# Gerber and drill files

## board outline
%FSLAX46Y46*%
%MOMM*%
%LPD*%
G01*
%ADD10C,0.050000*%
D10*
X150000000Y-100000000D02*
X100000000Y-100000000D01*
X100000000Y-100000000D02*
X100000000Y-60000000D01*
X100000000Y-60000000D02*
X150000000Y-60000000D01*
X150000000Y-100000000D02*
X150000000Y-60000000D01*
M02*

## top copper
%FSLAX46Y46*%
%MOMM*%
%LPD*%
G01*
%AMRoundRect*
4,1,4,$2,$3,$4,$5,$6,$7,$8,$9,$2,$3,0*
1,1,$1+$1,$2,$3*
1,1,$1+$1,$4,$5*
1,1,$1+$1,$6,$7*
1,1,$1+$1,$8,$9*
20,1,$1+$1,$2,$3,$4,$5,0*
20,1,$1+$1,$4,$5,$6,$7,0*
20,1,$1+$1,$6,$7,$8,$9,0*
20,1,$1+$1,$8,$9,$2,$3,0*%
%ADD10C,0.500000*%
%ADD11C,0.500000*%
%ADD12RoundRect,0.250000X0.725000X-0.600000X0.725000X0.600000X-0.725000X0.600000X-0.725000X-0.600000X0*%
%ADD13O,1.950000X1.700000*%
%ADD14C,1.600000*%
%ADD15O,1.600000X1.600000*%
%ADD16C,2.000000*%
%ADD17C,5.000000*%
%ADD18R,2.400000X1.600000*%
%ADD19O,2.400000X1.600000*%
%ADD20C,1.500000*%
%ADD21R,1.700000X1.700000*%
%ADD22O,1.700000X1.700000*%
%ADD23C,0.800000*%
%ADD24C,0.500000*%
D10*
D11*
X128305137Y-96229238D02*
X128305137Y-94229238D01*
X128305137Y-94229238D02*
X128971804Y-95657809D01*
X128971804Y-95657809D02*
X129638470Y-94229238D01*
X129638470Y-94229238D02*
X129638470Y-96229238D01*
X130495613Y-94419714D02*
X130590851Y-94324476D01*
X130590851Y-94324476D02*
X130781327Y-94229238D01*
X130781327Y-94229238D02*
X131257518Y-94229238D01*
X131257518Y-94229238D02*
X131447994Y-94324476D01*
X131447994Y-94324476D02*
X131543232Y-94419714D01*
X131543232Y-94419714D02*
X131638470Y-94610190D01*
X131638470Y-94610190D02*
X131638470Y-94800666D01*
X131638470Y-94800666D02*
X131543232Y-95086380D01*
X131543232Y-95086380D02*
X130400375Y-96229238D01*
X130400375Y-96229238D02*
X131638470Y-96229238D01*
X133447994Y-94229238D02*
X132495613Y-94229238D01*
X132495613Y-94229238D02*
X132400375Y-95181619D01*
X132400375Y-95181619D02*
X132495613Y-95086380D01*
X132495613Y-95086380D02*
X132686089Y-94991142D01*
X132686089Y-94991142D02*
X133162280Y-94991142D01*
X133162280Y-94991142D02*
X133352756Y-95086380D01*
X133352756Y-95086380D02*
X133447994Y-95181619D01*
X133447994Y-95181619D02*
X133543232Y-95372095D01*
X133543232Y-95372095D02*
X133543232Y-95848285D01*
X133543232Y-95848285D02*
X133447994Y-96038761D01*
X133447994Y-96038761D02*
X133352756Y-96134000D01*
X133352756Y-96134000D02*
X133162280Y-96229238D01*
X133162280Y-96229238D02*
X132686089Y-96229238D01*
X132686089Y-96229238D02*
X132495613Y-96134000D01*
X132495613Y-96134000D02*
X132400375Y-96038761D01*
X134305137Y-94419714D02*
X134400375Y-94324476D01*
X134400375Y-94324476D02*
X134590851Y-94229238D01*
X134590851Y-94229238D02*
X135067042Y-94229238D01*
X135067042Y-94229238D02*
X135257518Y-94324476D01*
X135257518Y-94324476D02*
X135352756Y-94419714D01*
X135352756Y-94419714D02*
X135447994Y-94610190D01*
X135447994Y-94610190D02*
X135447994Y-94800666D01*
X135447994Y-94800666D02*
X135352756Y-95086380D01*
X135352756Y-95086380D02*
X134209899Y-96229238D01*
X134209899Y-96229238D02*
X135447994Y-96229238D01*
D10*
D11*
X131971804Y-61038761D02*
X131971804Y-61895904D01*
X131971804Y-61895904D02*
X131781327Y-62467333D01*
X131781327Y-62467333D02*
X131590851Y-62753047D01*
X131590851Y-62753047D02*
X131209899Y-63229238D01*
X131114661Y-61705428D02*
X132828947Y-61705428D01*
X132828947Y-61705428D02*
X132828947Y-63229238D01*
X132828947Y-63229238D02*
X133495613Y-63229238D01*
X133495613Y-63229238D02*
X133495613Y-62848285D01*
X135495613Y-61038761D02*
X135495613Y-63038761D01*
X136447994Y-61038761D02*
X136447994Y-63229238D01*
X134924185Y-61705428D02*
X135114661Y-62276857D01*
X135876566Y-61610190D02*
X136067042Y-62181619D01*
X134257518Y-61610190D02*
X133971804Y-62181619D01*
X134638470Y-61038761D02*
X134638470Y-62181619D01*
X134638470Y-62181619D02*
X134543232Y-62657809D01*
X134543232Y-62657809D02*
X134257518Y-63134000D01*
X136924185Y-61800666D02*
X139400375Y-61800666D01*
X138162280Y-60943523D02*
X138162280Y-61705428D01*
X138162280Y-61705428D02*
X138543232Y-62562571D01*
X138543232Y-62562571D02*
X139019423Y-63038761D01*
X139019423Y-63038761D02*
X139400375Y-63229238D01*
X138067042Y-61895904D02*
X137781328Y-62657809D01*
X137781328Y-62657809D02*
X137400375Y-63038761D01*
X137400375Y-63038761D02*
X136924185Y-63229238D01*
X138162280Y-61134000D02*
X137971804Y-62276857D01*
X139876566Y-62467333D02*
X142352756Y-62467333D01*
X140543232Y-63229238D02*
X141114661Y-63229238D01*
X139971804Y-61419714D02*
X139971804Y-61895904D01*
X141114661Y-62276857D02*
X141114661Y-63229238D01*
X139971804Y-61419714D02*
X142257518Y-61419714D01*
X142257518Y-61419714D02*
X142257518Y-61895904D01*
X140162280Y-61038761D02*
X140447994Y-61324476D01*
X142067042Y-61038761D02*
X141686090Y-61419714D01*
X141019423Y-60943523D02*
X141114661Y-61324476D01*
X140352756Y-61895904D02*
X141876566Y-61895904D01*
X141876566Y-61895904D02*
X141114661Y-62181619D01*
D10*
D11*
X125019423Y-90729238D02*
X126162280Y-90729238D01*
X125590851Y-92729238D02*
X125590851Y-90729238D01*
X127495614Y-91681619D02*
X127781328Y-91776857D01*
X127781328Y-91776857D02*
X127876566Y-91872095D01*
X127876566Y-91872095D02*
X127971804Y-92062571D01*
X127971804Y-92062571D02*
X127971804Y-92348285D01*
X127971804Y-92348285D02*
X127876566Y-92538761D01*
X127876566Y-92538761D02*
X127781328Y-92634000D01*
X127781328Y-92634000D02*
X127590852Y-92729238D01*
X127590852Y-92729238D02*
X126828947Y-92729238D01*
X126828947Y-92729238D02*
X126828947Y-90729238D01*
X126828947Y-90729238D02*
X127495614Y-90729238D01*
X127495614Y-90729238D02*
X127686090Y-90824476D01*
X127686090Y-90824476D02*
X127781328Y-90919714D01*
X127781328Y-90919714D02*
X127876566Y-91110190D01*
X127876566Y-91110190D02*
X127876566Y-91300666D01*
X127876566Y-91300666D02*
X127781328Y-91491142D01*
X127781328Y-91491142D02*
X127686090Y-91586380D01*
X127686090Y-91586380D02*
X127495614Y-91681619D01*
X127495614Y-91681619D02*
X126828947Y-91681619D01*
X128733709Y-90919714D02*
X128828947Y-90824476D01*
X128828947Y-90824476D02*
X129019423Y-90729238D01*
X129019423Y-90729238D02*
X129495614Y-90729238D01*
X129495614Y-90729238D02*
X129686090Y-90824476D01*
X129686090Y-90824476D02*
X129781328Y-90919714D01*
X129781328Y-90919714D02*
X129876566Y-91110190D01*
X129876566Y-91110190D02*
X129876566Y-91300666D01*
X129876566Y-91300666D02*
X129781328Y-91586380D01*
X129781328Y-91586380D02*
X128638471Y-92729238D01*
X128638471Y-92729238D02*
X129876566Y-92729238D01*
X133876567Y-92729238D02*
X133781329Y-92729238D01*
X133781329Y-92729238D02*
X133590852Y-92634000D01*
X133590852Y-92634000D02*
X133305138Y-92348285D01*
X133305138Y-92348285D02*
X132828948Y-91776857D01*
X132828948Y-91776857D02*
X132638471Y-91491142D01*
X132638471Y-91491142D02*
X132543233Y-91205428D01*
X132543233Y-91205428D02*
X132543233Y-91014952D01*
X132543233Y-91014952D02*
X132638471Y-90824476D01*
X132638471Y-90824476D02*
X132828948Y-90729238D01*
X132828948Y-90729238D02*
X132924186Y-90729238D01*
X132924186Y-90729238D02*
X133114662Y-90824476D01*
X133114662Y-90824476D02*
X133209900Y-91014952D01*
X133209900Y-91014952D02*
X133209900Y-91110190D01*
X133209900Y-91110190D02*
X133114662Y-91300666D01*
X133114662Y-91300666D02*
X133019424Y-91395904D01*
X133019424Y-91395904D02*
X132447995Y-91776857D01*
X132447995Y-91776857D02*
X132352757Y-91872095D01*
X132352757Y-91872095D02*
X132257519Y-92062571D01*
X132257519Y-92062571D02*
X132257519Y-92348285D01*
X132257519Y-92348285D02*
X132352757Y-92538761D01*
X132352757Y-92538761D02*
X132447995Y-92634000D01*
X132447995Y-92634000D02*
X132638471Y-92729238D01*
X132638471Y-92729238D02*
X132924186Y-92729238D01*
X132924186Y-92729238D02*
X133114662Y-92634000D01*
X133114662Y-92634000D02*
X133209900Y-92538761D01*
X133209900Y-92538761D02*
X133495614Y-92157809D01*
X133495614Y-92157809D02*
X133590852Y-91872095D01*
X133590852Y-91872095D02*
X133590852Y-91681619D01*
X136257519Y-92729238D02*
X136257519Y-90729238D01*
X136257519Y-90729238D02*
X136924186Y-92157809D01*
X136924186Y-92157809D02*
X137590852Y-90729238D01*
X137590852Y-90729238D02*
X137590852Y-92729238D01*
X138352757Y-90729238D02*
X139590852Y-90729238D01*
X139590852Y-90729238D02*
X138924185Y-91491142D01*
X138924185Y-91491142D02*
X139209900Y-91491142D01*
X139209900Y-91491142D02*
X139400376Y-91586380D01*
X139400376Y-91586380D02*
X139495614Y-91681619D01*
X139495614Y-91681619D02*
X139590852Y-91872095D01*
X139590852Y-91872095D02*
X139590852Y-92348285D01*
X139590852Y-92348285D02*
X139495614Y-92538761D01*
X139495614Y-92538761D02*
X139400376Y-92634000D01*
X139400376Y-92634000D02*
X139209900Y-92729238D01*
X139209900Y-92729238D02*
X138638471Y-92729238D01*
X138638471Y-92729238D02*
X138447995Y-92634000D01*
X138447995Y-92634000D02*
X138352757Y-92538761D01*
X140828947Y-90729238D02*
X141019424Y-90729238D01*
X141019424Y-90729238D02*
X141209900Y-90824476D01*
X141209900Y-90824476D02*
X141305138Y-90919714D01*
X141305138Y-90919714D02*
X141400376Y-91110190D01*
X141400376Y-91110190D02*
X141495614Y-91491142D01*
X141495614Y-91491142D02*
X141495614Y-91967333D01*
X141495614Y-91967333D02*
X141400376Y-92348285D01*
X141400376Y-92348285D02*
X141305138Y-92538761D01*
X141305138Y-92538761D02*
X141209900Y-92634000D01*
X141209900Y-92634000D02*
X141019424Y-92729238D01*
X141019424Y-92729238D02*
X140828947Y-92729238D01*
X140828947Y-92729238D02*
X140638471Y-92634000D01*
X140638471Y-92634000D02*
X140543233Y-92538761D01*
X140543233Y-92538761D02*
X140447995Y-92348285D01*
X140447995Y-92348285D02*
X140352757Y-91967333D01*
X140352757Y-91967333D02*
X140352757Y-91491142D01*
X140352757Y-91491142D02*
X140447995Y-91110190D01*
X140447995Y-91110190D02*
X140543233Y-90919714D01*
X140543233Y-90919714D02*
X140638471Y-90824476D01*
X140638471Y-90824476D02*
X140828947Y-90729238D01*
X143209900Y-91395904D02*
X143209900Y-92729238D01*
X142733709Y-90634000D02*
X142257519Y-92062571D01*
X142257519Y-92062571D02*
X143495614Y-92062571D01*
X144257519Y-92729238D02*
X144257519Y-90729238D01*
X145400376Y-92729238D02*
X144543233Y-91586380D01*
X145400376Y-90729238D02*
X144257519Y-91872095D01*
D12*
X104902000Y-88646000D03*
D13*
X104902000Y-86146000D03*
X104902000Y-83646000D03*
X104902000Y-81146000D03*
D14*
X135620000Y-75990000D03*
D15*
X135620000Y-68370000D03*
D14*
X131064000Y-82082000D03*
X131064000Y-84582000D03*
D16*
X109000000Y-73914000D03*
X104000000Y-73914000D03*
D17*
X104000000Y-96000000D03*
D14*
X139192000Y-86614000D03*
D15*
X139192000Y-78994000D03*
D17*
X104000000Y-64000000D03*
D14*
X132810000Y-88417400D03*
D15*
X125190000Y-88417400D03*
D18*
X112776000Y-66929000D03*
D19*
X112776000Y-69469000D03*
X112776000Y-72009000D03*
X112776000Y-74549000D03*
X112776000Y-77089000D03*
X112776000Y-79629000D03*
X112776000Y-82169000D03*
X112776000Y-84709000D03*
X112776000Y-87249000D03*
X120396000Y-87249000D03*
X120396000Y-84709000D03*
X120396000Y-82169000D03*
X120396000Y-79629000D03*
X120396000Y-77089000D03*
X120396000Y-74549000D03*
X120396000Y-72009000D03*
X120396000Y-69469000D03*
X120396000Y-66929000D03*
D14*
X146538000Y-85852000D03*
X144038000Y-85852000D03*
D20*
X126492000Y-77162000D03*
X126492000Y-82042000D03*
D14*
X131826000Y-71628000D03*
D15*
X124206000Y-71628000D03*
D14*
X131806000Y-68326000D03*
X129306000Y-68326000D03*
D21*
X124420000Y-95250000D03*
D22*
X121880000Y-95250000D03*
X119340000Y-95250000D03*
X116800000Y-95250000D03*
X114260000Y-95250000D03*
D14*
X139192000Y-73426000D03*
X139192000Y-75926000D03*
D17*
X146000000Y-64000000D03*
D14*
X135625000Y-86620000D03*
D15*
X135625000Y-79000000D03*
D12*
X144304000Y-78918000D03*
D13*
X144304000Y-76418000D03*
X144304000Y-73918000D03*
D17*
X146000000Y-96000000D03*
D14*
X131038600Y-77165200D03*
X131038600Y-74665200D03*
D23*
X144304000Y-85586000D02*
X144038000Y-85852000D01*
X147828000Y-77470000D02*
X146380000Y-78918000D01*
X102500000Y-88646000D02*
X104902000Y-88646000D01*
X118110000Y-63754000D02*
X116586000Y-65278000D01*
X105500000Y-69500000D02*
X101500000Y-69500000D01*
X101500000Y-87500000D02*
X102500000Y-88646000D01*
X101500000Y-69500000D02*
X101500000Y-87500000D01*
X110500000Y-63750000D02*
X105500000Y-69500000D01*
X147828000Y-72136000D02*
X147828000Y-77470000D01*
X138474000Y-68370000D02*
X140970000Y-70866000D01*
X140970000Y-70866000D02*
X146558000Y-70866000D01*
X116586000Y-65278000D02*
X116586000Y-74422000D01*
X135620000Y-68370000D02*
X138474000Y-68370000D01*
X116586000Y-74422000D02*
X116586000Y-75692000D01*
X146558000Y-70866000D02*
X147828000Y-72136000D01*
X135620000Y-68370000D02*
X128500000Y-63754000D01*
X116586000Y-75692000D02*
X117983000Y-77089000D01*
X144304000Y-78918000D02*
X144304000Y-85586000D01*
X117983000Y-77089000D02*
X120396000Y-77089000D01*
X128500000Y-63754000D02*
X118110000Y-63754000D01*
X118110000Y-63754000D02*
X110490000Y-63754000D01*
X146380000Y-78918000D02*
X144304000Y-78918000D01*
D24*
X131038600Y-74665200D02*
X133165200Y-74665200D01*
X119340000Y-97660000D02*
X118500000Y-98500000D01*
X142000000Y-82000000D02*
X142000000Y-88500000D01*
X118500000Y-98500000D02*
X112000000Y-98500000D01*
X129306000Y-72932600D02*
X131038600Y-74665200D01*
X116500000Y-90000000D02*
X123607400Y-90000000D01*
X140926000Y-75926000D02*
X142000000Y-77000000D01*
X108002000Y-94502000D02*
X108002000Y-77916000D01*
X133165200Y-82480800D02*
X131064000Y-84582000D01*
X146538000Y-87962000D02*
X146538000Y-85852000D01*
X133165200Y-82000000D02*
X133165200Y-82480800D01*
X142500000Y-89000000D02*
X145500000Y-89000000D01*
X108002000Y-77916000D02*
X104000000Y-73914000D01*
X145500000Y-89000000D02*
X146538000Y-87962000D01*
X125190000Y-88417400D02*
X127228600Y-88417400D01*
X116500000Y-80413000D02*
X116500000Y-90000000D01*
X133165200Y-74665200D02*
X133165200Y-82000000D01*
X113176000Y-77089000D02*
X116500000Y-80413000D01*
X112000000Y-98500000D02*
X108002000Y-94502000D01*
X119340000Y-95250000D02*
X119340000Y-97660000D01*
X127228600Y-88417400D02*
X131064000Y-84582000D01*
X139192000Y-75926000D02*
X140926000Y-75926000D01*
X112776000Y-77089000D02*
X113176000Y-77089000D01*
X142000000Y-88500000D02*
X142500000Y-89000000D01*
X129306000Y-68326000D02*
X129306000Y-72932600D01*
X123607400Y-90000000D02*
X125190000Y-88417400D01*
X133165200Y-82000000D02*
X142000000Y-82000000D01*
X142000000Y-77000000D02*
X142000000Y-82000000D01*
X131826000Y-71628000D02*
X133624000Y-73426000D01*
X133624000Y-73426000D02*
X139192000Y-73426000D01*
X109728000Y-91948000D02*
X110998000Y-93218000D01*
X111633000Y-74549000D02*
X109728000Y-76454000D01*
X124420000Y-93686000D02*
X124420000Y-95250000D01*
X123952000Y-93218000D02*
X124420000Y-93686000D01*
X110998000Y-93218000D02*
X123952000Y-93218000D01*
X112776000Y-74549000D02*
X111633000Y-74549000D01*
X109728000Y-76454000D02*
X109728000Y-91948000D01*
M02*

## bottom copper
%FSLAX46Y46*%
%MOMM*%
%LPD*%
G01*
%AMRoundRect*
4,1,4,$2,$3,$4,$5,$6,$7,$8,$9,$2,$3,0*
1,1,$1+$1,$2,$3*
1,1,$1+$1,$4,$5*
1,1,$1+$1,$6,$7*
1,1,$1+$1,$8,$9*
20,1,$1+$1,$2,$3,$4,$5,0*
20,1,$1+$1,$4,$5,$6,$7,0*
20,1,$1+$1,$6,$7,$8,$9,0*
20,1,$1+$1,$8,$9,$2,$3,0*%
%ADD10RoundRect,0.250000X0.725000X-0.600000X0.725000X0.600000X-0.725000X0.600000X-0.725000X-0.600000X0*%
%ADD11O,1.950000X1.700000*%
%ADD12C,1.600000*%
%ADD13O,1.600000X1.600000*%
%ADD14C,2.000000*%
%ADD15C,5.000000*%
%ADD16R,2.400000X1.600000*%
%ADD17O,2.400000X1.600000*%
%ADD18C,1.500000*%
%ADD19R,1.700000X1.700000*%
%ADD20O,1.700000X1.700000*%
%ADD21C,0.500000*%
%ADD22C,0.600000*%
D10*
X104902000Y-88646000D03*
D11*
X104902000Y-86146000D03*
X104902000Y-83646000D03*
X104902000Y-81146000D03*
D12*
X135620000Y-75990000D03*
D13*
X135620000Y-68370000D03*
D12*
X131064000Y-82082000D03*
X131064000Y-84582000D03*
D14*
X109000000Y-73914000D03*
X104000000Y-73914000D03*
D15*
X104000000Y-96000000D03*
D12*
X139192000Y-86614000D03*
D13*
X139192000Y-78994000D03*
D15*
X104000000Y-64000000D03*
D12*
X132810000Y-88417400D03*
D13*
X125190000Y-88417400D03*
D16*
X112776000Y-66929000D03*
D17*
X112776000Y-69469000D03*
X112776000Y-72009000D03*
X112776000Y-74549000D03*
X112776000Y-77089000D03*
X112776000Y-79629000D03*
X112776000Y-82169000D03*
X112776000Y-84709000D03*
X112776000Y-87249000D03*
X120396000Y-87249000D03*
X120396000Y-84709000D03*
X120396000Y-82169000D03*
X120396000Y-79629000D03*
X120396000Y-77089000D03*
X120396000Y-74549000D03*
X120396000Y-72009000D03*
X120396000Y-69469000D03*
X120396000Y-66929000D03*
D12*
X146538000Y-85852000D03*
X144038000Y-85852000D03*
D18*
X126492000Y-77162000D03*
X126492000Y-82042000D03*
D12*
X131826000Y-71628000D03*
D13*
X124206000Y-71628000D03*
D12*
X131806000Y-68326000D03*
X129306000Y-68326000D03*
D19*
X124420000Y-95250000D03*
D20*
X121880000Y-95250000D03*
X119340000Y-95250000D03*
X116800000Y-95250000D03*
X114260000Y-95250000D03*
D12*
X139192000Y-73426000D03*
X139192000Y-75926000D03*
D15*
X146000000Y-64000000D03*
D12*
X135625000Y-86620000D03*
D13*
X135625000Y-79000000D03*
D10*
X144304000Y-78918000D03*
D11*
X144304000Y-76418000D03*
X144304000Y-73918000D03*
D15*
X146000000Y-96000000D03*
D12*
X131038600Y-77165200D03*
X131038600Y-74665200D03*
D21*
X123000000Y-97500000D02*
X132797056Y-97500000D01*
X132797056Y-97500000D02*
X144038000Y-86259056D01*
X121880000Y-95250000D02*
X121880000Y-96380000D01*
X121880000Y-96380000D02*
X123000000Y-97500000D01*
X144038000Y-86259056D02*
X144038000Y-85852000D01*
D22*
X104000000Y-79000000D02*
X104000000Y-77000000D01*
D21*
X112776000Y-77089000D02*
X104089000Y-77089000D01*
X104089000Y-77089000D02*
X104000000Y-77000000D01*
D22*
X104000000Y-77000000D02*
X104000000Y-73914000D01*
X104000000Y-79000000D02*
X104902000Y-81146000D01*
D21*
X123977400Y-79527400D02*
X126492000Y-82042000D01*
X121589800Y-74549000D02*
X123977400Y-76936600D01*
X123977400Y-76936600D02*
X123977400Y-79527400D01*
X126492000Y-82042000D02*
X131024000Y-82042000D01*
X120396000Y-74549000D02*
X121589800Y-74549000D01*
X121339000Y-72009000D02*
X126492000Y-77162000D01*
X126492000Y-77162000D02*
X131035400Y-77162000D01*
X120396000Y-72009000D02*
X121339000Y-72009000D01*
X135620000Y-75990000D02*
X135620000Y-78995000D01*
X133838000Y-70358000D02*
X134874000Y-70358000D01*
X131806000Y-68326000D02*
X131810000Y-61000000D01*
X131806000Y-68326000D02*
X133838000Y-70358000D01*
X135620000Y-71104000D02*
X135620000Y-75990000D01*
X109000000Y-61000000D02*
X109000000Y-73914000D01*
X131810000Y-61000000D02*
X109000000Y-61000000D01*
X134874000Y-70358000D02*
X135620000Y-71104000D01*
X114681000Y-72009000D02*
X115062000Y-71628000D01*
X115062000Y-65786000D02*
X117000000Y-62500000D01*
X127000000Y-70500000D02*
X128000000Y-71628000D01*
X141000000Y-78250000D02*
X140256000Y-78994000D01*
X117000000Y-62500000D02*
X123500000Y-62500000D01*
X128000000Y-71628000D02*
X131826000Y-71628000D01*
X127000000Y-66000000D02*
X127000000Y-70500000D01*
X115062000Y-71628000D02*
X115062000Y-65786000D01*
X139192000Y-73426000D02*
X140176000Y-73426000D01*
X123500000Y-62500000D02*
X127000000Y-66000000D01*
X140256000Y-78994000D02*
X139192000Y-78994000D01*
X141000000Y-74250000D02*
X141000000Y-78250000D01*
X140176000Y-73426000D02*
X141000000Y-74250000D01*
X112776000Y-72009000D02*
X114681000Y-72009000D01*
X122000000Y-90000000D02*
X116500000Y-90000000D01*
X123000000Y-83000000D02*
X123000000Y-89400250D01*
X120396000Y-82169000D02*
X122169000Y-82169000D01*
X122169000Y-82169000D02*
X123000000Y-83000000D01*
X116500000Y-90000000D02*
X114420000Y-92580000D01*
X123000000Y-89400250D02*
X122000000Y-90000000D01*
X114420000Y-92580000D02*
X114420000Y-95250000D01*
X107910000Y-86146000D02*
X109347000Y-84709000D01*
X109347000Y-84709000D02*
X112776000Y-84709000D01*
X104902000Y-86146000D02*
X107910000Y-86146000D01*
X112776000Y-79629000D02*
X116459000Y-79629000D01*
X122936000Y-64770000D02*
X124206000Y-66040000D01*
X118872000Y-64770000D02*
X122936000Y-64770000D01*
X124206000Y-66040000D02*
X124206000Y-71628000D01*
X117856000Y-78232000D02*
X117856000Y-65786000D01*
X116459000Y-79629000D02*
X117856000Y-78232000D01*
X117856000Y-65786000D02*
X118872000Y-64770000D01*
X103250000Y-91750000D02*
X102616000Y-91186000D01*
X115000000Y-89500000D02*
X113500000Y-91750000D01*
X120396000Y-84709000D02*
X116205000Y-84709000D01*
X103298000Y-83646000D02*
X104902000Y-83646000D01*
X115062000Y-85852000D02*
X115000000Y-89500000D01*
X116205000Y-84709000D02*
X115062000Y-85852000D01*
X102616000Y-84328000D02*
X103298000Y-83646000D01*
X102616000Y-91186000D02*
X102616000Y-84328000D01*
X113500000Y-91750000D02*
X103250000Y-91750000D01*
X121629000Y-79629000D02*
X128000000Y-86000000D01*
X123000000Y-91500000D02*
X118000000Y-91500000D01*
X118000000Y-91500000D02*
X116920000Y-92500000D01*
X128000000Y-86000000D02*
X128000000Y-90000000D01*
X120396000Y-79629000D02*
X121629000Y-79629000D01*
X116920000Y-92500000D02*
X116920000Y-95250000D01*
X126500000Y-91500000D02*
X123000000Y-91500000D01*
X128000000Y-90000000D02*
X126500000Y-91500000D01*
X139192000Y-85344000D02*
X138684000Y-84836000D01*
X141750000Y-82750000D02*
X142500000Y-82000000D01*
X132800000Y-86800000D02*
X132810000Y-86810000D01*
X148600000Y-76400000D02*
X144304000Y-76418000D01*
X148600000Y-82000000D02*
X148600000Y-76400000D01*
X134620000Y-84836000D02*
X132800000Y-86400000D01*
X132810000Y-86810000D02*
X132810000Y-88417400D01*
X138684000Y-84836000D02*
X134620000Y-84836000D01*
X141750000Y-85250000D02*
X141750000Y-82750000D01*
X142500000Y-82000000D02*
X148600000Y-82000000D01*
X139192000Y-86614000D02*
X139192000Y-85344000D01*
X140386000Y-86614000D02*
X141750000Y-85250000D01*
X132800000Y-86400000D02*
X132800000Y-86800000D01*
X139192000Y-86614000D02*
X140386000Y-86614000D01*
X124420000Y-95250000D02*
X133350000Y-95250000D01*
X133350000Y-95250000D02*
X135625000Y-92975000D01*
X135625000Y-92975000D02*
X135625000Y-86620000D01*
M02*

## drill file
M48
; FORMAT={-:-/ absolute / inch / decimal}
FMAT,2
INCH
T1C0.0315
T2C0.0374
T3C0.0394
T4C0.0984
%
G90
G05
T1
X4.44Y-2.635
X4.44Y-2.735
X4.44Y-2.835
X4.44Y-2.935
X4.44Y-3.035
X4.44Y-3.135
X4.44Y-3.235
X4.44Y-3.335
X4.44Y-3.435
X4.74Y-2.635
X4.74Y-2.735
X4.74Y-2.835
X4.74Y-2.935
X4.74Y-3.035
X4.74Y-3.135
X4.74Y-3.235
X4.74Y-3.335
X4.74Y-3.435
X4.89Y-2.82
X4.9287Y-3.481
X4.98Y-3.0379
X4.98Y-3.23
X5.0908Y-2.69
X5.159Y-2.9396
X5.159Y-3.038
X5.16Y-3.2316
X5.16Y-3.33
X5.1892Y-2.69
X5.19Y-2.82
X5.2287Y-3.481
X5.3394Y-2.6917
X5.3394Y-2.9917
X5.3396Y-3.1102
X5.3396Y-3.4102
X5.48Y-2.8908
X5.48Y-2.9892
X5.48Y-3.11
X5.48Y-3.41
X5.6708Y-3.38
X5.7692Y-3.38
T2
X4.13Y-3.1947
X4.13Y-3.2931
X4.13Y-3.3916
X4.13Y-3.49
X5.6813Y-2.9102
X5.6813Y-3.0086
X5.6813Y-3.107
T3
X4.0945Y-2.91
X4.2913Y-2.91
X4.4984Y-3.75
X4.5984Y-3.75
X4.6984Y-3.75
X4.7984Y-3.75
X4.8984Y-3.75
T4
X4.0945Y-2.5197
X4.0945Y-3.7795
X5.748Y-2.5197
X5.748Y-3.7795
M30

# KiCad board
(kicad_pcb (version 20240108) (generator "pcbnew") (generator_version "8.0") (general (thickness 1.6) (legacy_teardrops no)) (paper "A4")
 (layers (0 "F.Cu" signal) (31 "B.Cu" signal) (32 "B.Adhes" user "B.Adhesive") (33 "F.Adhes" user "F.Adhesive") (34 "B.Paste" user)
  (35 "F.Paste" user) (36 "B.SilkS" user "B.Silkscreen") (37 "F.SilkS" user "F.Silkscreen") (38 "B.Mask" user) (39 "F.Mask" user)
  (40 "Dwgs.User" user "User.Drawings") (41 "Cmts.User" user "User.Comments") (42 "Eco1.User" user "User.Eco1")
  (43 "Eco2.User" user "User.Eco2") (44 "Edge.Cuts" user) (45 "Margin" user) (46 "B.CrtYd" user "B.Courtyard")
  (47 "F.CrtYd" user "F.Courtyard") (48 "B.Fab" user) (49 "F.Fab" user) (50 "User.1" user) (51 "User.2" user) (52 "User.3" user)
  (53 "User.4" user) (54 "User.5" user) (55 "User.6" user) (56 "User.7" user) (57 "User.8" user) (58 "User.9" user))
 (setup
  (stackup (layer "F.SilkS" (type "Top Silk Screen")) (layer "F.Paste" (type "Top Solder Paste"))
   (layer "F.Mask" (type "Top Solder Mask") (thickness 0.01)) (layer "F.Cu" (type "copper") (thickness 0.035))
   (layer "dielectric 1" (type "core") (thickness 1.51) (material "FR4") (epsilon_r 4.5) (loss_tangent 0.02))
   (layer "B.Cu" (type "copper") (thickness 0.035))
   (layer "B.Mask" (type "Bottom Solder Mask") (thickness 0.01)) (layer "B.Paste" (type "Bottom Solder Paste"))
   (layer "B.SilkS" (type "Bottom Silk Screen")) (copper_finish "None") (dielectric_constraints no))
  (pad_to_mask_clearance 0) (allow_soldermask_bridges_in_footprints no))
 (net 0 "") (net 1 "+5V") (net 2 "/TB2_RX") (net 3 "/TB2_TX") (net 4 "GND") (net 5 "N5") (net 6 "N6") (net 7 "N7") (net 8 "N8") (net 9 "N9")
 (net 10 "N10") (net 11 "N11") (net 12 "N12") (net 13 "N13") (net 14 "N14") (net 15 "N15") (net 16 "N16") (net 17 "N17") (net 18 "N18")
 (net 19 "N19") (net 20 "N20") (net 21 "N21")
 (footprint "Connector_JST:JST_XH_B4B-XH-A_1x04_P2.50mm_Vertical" (layer "F.Cu") (at 104.902 88.646 90)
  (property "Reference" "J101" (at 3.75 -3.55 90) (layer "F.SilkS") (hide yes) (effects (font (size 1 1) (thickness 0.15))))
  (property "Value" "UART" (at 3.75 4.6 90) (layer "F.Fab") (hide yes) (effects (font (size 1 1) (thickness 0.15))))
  (pad "1" thru_hole roundrect (at 0 0 90) (size 1.7 1.95) (drill 0.95) (layers "*.Cu" "*.Mask") (remove_unused_layers no)
   (roundrect_rratio 0.147059) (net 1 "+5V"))
  (pad "2" thru_hole oval (at 2.5 0 90) (size 1.7 1.95) (drill 0.95) (layers "*.Cu" "*.Mask") (remove_unused_layers no) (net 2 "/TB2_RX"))
  (pad "3" thru_hole oval (at 5 0 90) (size 1.7 1.95) (drill 0.95) (layers "*.Cu" "*.Mask") (remove_unused_layers no) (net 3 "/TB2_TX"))
  (pad "4" thru_hole oval (at 7.5 0 90) (size 1.7 1.95) (drill 0.95) (layers "*.Cu" "*.Mask") (remove_unused_layers no) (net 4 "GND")))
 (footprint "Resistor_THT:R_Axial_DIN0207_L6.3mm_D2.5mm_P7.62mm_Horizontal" (layer "F.Cu") (at 135.62 75.99 90)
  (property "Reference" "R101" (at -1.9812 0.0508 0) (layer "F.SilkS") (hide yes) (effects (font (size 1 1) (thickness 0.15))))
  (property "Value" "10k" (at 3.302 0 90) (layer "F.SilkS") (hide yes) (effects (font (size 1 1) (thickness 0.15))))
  (pad "1" thru_hole circle (at 0 0 90) (size 1.6 1.6) (drill 0.8) (layers "*.Cu" "*.Mask") (remove_unused_layers no) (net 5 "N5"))
  (pad "2" thru_hole oval (at 7.62 0 90) (size 1.6 1.6) (drill 0.8) (layers "*.Cu" "*.Mask") (remove_unused_layers no) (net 1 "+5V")))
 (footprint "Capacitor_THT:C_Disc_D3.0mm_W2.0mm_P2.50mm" (layer "F.Cu") (at 131.064 82.082 -90)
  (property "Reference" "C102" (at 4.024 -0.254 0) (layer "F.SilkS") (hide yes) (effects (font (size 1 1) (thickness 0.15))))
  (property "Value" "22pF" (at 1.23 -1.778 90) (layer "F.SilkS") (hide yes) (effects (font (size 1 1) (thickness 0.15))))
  (pad "1" thru_hole circle (at 0 0 270) (size 1.6 1.6) (drill 0.8) (layers "*.Cu" "*.Mask") (remove_unused_layers no) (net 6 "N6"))
  (pad "2" thru_hole circle (at 2.5 0 270) (size 1.6 1.6) (drill 0.8) (layers "*.Cu" "*.Mask") (remove_unused_layers no) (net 4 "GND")))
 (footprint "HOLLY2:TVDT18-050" (layer "F.Cu") (at 106.5 73.914 180)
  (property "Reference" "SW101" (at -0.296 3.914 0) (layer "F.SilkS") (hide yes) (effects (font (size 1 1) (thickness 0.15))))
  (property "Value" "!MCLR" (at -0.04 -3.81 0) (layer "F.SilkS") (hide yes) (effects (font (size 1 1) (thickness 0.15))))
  (pad "1" thru_hole circle (at -2.5 0 180) (size 2 2) (drill 1) (layers "*.Cu" "*.Mask") (remove_unused_layers no) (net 5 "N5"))
  (pad "2" thru_hole circle (at 2.5 0 180) (size 2 2) (drill 1) (layers "*.Cu" "*.Mask") (remove_unused_layers no) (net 4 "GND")))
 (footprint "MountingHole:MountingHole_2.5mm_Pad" (layer "F.Cu") (at 104 96)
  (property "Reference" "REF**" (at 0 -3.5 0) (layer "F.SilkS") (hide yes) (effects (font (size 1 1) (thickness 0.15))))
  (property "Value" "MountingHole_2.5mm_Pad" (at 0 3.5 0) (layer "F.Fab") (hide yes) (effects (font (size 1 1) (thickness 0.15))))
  (pad "" np_thru_hole circle (at 0 0) (size 5 5) (drill 2.5) (layers "F&B.Cu" "*.Mask")))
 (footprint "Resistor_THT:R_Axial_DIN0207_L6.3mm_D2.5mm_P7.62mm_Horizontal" (layer "F.Cu") (at 139.192 86.614 90)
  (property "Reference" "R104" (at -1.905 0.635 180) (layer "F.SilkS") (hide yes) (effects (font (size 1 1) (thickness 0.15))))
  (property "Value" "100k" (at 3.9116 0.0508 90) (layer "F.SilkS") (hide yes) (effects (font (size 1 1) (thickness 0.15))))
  (pad "1" thru_hole circle (at 0 0 90) (size 1.6 1.6) (drill 0.8) (layers "*.Cu" "*.Mask") (remove_unused_layers no) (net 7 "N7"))
  (pad "2" thru_hole oval (at 7.62 0 90) (size 1.6 1.6) (drill 0.8) (layers "*.Cu" "*.Mask") (remove_unused_layers no) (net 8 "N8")))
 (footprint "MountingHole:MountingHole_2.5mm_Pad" (layer "F.Cu") (at 104 64)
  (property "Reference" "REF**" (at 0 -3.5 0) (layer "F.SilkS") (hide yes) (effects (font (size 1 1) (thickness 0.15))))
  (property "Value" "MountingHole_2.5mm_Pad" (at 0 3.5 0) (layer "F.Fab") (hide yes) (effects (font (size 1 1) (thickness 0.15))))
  (pad "" np_thru_hole circle (at 0 0) (size 5 5) (drill 2.5) (layers "F&B.Cu" "*.Mask")))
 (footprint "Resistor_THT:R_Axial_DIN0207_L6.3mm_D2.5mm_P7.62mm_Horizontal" (layer "F.Cu") (at 132.81 88.4174 180)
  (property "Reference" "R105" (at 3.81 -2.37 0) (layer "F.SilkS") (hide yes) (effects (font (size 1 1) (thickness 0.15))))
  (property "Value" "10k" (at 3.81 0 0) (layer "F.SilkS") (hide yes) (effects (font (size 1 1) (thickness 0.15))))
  (pad "1" thru_hole circle (at 0 0 180) (size 1.6 1.6) (drill 0.8) (layers "*.Cu" "*.Mask") (remove_unused_layers no) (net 7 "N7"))
  (pad "2" thru_hole oval (at 7.62 0 180) (size 1.6 1.6) (drill 0.8) (layers "*.Cu" "*.Mask") (remove_unused_layers no) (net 4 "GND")))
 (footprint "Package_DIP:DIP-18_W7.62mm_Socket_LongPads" (layer "F.Cu") (at 112.776 66.929)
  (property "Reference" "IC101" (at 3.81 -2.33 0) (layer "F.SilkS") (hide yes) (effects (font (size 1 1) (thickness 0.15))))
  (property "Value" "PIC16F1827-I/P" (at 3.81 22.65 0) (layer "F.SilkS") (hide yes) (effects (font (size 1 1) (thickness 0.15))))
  (pad "1" thru_hole rect (at 0 0) (size 2.4 1.6) (drill 0.8) (layers "*.Cu" "*.Mask") (remove_unused_layers no) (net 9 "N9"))
  (pad "2" thru_hole oval (at 0 2.54) (size 2.4 1.6) (drill 0.8) (layers "*.Cu" "*.Mask") (remove_unused_layers no) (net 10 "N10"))
  (pad "3" thru_hole oval (at 0 5.08) (size 2.4 1.6) (drill 0.8) (layers "*.Cu" "*.Mask") (remove_unused_layers no) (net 8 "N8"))
  (pad "4" thru_hole oval (at 0 7.62) (size 2.4 1.6) (drill 0.8) (layers "*.Cu" "*.Mask") (remove_unused_layers no) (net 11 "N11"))
  (pad "5" thru_hole oval (at 0 10.16) (size 2.4 1.6) (drill 0.8) (layers "*.Cu" "*.Mask") (remove_unused_layers no) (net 4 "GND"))
  (pad "6" thru_hole oval (at 0 12.7) (size 2.4 1.6) (drill 0.8) (layers "*.Cu" "*.Mask") (remove_unused_layers no) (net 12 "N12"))
  (pad "7" thru_hole oval (at 0 15.24) (size 2.4 1.6) (drill 0.8) (layers "*.Cu" "*.Mask") (remove_unused_layers no) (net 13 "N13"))
  (pad "8" thru_hole oval (at 0 17.78) (size 2.4 1.6) (drill 0.8) (layers "*.Cu" "*.Mask") (remove_unused_layers no) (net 2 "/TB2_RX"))
  (pad "9" thru_hole oval (at 0 20.32) (size 2.4 1.6) (drill 0.8) (layers "*.Cu" "*.Mask") (remove_unused_layers no) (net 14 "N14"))
  (pad "10" thru_hole oval (at 7.62 20.32) (size 2.4 1.6) (drill 0.8) (layers "*.Cu" "*.Mask") (remove_unused_layers no) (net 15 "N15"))
  (pad "11" thru_hole oval (at 7.62 17.78) (size 2.4 1.6) (drill 0.8) (layers "*.Cu" "*.Mask") (remove_unused_layers no) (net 3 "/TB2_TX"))
  (pad "12" thru_hole oval (at 7.62 15.24) (size 2.4 1.6) (drill 0.8) (layers "*.Cu" "*.Mask") (remove_unused_layers no) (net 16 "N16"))
  (pad "13" thru_hole oval (at 7.62 12.7) (size 2.4 1.6) (drill 0.8) (layers "*.Cu" "*.Mask") (remove_unused_layers no) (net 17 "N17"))
  (pad "14" thru_hole oval (at 7.62 10.16) (size 2.4 1.6) (drill 0.8) (layers "*.Cu" "*.Mask") (remove_unused_layers no) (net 1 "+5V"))
  (pad "15" thru_hole oval (at 7.62 7.62) (size 2.4 1.6) (drill 0.8) (layers "*.Cu" "*.Mask") (remove_unused_layers no) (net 6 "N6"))
  (pad "16" thru_hole oval (at 7.62 5.08) (size 2.4 1.6) (drill 0.8) (layers "*.Cu" "*.Mask") (remove_unused_layers no) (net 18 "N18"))
  (pad "17" thru_hole oval (at 7.62 2.54) (size 2.4 1.6) (drill 0.8) (layers "*.Cu" "*.Mask") (remove_unused_layers no) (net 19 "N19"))
  (pad "18" thru_hole oval (at 7.62 0) (size 2.4 1.6) (drill 0.8) (layers "*.Cu" "*.Mask") (remove_unused_layers no) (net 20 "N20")))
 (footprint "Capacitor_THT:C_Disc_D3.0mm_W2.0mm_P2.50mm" (layer "F.Cu") (at 146.538 85.852 180)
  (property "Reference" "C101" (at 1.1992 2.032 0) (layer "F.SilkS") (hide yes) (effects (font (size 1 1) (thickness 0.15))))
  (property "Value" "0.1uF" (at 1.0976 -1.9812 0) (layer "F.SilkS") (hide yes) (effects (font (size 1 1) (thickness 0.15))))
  (pad "1" thru_hole circle (at 0 0 180) (size 1.6 1.6) (drill 0.8) (layers "*.Cu" "*.Mask") (remove_unused_layers no) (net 4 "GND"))
  (pad "2" thru_hole circle (at 2.5 0 180) (size 1.6 1.6) (drill 0.8) (layers "*.Cu" "*.Mask") (remove_unused_layers no) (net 1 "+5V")))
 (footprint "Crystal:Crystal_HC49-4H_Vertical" (layer "F.Cu") (at 126.492 77.162 -90)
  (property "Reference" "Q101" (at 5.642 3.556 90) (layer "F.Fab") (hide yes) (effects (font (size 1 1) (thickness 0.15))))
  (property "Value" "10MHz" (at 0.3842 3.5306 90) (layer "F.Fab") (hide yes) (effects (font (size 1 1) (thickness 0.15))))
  (pad "1" thru_hole circle (at 0 0 270) (size 1.5 1.5) (drill 0.8) (layers "*.Cu" "*.Mask") (remove_unused_layers no) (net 18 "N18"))
  (pad "2" thru_hole circle (at 4.88 0 270) (size 1.5 1.5) (drill 0.8) (layers "*.Cu" "*.Mask") (remove_unused_layers no) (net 6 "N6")))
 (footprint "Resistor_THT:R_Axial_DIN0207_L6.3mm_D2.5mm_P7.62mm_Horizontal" (layer "F.Cu") (at 131.826 71.628 180)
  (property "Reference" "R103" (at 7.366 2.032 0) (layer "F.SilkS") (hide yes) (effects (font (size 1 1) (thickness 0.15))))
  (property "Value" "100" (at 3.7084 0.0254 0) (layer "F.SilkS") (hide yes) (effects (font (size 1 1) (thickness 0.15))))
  (pad "1" thru_hole circle (at 0 0 180) (size 1.6 1.6) (drill 0.8) (layers "*.Cu" "*.Mask") (remove_unused_layers no) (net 8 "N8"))
  (pad "2" thru_hole oval (at 7.62 0 180) (size 1.6 1.6) (drill 0.8) (layers "*.Cu" "*.Mask") (remove_unused_layers no) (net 12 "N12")))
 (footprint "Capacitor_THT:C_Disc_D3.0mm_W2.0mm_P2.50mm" (layer "F.Cu") (at 131.806 68.326 180)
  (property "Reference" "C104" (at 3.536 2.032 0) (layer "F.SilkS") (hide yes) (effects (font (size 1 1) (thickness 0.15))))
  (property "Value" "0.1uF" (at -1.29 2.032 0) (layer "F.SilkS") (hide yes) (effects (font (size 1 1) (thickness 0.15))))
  (pad "1" thru_hole circle (at 0 0 180) (size 1.6 1.6) (drill 0.8) (layers "*.Cu" "*.Mask") (remove_unused_layers no) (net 5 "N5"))
  (pad "2" thru_hole circle (at 2.5 0 180) (size 1.6 1.6) (drill 0.8) (layers "*.Cu" "*.Mask") (remove_unused_layers no) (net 4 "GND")))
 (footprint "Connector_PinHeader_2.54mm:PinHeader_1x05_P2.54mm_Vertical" (layer "F.Cu") (at 124.42 95.25 -90)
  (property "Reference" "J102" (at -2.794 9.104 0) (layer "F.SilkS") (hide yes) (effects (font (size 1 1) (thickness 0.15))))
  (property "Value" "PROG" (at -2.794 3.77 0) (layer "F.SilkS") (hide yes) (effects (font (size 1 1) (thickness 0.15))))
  (pad "1" thru_hole rect (at 0 0 270) (size 1.7 1.7) (drill 1) (layers "*.Cu" "*.Mask") (remove_unused_layers no) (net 11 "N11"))
  (pad "2" thru_hole oval (at 0 2.54 270) (size 1.7 1.7) (drill 1) (layers "*.Cu" "*.Mask") (remove_unused_layers no) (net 1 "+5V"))
  (pad "3" thru_hole oval (at 0 5.08 270) (size 1.7 1.7) (drill 1) (layers "*.Cu" "*.Mask") (remove_unused_layers no) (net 4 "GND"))
  (pad "4" thru_hole oval (at 0 7.62 270) (size 1.7 1.7) (drill 1) (layers "*.Cu" "*.Mask") (remove_unused_layers no) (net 17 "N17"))
  (pad "5" thru_hole oval (at 0 10.16 270) (size 1.7 1.7) (drill 1) (layers "*.Cu" "*.Mask") (remove_unused_layers no) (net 16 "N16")))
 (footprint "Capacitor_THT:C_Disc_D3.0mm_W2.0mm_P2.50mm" (layer "F.Cu") (at 139.192 73.426 -90)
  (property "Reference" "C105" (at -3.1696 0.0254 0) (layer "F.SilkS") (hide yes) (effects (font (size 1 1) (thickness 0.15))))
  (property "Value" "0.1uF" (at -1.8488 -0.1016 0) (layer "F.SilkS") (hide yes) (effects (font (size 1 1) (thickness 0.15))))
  (pad "1" thru_hole circle (at 0 0 270) (size 1.6 1.6) (drill 0.8) (layers "*.Cu" "*.Mask") (remove_unused_layers no) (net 8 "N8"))
  (pad "2" thru_hole circle (at 2.5 0 270) (size 1.6 1.6) (drill 0.8) (layers "*.Cu" "*.Mask") (remove_unused_layers no) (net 4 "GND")))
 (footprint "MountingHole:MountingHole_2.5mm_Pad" (layer "F.Cu") (at 146 64)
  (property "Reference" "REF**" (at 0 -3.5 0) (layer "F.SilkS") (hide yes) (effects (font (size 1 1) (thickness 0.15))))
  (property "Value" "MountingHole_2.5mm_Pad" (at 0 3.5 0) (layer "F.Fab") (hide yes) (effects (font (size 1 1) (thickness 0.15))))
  (pad "" np_thru_hole circle (at 0 0) (size 5 5) (drill 2.5) (layers "F&B.Cu" "*.Mask")))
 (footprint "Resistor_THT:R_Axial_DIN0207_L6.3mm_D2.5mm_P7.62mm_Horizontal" (layer "F.Cu") (at 135.625 86.62 90)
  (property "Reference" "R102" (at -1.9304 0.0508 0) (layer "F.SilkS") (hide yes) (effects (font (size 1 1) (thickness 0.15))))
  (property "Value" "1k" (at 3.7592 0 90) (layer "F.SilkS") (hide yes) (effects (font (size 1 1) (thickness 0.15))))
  (pad "1" thru_hole circle (at 0 0 90) (size 1.6 1.6) (drill 0.8) (layers "*.Cu" "*.Mask") (remove_unused_layers no) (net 11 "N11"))
  (pad "2" thru_hole oval (at 7.62 0 90) (size 1.6 1.6) (drill 0.8) (layers "*.Cu" "*.Mask") (remove_unused_layers no) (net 5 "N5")))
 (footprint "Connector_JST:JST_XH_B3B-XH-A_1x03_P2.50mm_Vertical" (layer "F.Cu") (at 144.304 78.918 90)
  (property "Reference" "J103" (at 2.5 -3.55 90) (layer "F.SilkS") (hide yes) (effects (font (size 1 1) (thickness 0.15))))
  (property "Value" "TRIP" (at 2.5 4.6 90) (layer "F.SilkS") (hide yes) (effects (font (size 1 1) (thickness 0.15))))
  (pad "1" thru_hole roundrect (at 0 0 90) (size 1.7 1.95) (drill 0.95) (layers "*.Cu" "*.Mask") (remove_unused_layers no)
   (roundrect_rratio 0.147059) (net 1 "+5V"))
  (pad "2" thru_hole oval (at 2.5 0 90) (size 1.7 1.95) (drill 0.95) (layers "*.Cu" "*.Mask") (remove_unused_layers no) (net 7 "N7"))
  (pad "3" thru_hole oval (at 5 0 90) (size 1.7 1.95) (drill 0.95) (layers "*.Cu" "*.Mask") (remove_unused_layers no) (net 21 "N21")))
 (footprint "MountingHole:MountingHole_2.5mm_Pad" (layer "F.Cu") (at 146 96)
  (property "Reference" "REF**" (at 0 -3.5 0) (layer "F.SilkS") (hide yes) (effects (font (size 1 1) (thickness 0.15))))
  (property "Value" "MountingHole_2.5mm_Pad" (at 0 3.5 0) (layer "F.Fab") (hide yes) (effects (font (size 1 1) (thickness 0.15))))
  (pad "" np_thru_hole circle (at 0 0) (size 5 5) (drill 2.5) (layers "F&B.Cu" "*.Mask")))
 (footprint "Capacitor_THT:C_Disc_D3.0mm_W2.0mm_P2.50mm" (layer "F.Cu") (at 131.0386 77.1652 90)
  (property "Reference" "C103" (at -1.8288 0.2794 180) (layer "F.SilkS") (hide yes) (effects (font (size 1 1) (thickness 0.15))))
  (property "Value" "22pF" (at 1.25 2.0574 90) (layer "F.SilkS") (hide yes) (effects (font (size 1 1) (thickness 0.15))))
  (pad "1" thru_hole circle (at 0 0 90) (size 1.6 1.6) (drill 0.8) (layers "*.Cu" "*.Mask") (remove_unused_layers no) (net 18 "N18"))
  (pad "2" thru_hole circle (at 2.5 0 90) (size 1.6 1.6) (drill 0.8) (layers "*.Cu" "*.Mask") (remove_unused_layers no) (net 4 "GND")))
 (gr_line (start 150 100) (end 100 100) (stroke (width 0.05) (type default)) (layer "Edge.Cuts"))
 (gr_line (start 100 100) (end 100 60) (stroke (width 0.05) (type default)) (layer "Edge.Cuts"))
 (gr_line (start 100 60) (end 150 60) (stroke (width 0.05) (type default)) (layer "Edge.Cuts"))
 (gr_line (start 150 100) (end 150 60) (stroke (width 0.05) (type default)) (layer "Edge.Cuts"))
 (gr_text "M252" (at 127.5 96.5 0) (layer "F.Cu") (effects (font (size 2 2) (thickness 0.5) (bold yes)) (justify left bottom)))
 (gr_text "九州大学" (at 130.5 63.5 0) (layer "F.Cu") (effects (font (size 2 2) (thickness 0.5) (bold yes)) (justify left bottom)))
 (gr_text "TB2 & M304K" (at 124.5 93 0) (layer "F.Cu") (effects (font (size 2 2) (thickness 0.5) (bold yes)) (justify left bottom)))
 (segment (start 144.304 85.586) (end 144.038 85.852) (width 0.8) (layer "F.Cu") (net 1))
 (segment (start 147.828 77.47) (end 146.38 78.918) (width 0.8) (layer "F.Cu") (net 1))
 (segment (start 102.5 88.646) (end 104.902 88.646) (width 0.8) (layer "F.Cu") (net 1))
 (segment (start 118.11 63.754) (end 116.586 65.278) (width 0.8) (layer "F.Cu") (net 1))
 (segment (start 105.5 69.5) (end 101.5 69.5) (width 0.8) (layer "F.Cu") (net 1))
 (segment (start 101.5 87.5) (end 102.5 88.646) (width 0.8) (layer "F.Cu") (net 1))
 (segment (start 101.5 69.5) (end 101.5 87.5) (width 0.8) (layer "F.Cu") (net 1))
 (segment (start 110.5 63.75) (end 105.5 69.5) (width 0.8) (layer "F.Cu") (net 1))
 (segment (start 147.828 72.136) (end 147.828 77.47) (width 0.8) (layer "F.Cu") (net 1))
 (segment (start 138.474 68.37) (end 140.97 70.866) (width 0.8) (layer "F.Cu") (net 1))
 (segment (start 140.97 70.866) (end 146.558 70.866) (width 0.8) (layer "F.Cu") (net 1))
 (segment (start 116.586 65.278) (end 116.586 74.422) (width 0.8) (layer "F.Cu") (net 1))
 (segment (start 135.62 68.37) (end 138.474 68.37) (width 0.8) (layer "F.Cu") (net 1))
 (segment (start 116.586 74.422) (end 116.586 75.692) (width 0.8) (layer "F.Cu") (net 1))
 (segment (start 146.558 70.866) (end 147.828 72.136) (width 0.8) (layer "F.Cu") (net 1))
 (segment (start 135.62 68.37) (end 128.5 63.754) (width 0.8) (layer "F.Cu") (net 1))
 (segment (start 116.586 75.692) (end 117.983 77.089) (width 0.8) (layer "F.Cu") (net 1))
 (segment (start 144.304 78.918) (end 144.304 85.586) (width 0.8) (layer "F.Cu") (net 1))
 (segment (start 117.983 77.089) (end 120.396 77.089) (width 0.8) (layer "F.Cu") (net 1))
 (segment (start 128.5 63.754) (end 118.11 63.754) (width 0.8) (layer "F.Cu") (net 1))
 (segment (start 118.11 63.754) (end 110.49 63.754) (width 0.8) (layer "F.Cu") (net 1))
 (segment (start 146.38 78.918) (end 144.304 78.918) (width 0.8) (layer "F.Cu") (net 1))
 (segment (start 123 97.5) (end 132.797056 97.5) (width 0.5) (layer "B.Cu") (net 1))
 (segment (start 132.797056 97.5) (end 144.038 86.259056) (width 0.5) (layer "B.Cu") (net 1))
 (segment (start 121.88 95.25) (end 121.88 96.38) (width 0.5) (layer "B.Cu") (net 1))
 (segment (start 121.88 96.38) (end 123 97.5) (width 0.5) (layer "B.Cu") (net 1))
 (segment (start 144.038 86.259056) (end 144.038 85.852) (width 0.5) (layer "B.Cu") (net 1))
 (segment (start 131.0386 74.6652) (end 133.1652 74.6652) (width 0.5) (layer "F.Cu") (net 4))
 (segment (start 119.34 97.66) (end 118.5 98.5) (width 0.5) (layer "F.Cu") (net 4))
 (segment (start 142 82) (end 142 88.5) (width 0.5) (layer "F.Cu") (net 4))
 (segment (start 118.5 98.5) (end 112 98.5) (width 0.5) (layer "F.Cu") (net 4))
 (segment (start 129.306 72.9326) (end 131.0386 74.6652) (width 0.5) (layer "F.Cu") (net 4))
 (segment (start 116.5 90) (end 123.6074 90) (width 0.5) (layer "F.Cu") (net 4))
 (segment (start 140.926 75.926) (end 142 77) (width 0.5) (layer "F.Cu") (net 4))
 (segment (start 108.002 94.502) (end 108.002 77.916) (width 0.5) (layer "F.Cu") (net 4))
 (segment (start 133.1652 82.4808) (end 131.064 84.582) (width 0.5) (layer "F.Cu") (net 4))
 (segment (start 146.538 87.962) (end 146.538 85.852) (width 0.5) (layer "F.Cu") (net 4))
 (segment (start 133.1652 82) (end 133.1652 82.4808) (width 0.5) (layer "F.Cu") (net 4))
 (segment (start 142.5 89) (end 145.5 89) (width 0.5) (layer "F.Cu") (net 4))
 (segment (start 108.002 77.916) (end 104 73.914) (width 0.5) (layer "F.Cu") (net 4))
 (segment (start 145.5 89) (end 146.538 87.962) (width 0.5) (layer "F.Cu") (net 4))
 (segment (start 125.19 88.4174) (end 127.2286 88.4174) (width 0.5) (layer "F.Cu") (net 4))
 (segment (start 116.5 80.413) (end 116.5 90) (width 0.5) (layer "F.Cu") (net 4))
 (segment (start 133.1652 74.6652) (end 133.1652 82) (width 0.5) (layer "F.Cu") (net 4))
 (segment (start 113.176 77.089) (end 116.5 80.413) (width 0.5) (layer "F.Cu") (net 4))
 (segment (start 112 98.5) (end 108.002 94.502) (width 0.5) (layer "F.Cu") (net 4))
 (segment (start 119.34 95.25) (end 119.34 97.66) (width 0.5) (layer "F.Cu") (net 4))
 (segment (start 127.2286 88.4174) (end 131.064 84.582) (width 0.5) (layer "F.Cu") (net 4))
 (segment (start 139.192 75.926) (end 140.926 75.926) (width 0.5) (layer "F.Cu") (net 4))
 (segment (start 112.776 77.089) (end 113.176 77.089) (width 0.5) (layer "F.Cu") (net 4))
 (segment (start 142 88.5) (end 142.5 89) (width 0.5) (layer "F.Cu") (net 4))
 (segment (start 129.306 68.326) (end 129.306 72.9326) (width 0.5) (layer "F.Cu") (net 4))
 (segment (start 123.6074 90) (end 125.19 88.4174) (width 0.5) (layer "F.Cu") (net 4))
 (segment (start 133.1652 82) (end 142 82) (width 0.5) (layer "F.Cu") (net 4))
 (segment (start 142 77) (end 142 82) (width 0.5) (layer "F.Cu") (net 4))
 (segment (start 104 79) (end 104 77) (width 0.6) (layer "B.Cu") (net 4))
 (segment (start 112.776 77.089) (end 104.089 77.089) (width 0.5) (layer "B.Cu") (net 4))
 (segment (start 104.089 77.089) (end 104 77) (width 0.5) (layer "B.Cu") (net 4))
 (segment (start 104 77) (end 104 73.914) (width 0.6) (layer "B.Cu") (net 4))
 (segment (start 104 79) (end 104.902 81.146) (width 0.6) (layer "B.Cu") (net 4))
 (segment (start 123.9774 79.5274) (end 126.492 82.042) (width 0.5) (layer "B.Cu") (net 6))
 (segment (start 121.5898 74.549) (end 123.9774 76.9366) (width 0.5) (layer "B.Cu") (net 6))
 (segment (start 123.9774 76.9366) (end 123.9774 79.5274) (width 0.5) (layer "B.Cu") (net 6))
 (segment (start 126.492 82.042) (end 131.024 82.042) (width 0.5) (layer "B.Cu") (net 6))
 (segment (start 120.396 74.549) (end 121.5898 74.549) (width 0.5) (layer "B.Cu") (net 6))
 (segment (start 121.339 72.009) (end 126.492 77.162) (width 0.5) (layer "B.Cu") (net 18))
 (segment (start 126.492 77.162) (end 131.0354 77.162) (width 0.5) (layer "B.Cu") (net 18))
 (segment (start 120.396 72.009) (end 121.339 72.009) (width 0.5) (layer "B.Cu") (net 18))
 (segment (start 135.62 75.99) (end 135.62 78.995) (width 0.5) (layer "B.Cu") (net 5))
 (segment (start 133.838 70.358) (end 134.874 70.358) (width 0.5) (layer "B.Cu") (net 5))
 (segment (start 131.806 68.326) (end 131.81 61) (width 0.5) (layer "B.Cu") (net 5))
 (segment (start 131.806 68.326) (end 133.838 70.358) (width 0.5) (layer "B.Cu") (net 5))
 (segment (start 135.62 71.104) (end 135.62 75.99) (width 0.5) (layer "B.Cu") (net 5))
 (segment (start 109 61) (end 109 73.914) (width 0.5) (layer "B.Cu") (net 5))
 (segment (start 131.81 61) (end 109 61) (width 0.5) (layer "B.Cu") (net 5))
 (segment (start 134.874 70.358) (end 135.62 71.104) (width 0.5) (layer "B.Cu") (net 5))
 (segment (start 131.826 71.628) (end 133.624 73.426) (width 0.5) (layer "F.Cu") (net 8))
 (segment (start 133.624 73.426) (end 139.192 73.426) (width 0.5) (layer "F.Cu") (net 8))
 (segment (start 114.681 72.009) (end 115.062 71.628) (width 0.5) (layer "B.Cu") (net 8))
 (segment (start 115.062 65.786) (end 117 62.5) (width 0.5) (layer "B.Cu") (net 8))
 (segment (start 127 70.5) (end 128 71.628) (width 0.5) (layer "B.Cu") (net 8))
 (segment (start 141 78.25) (end 140.256 78.994) (width 0.5) (layer "B.Cu") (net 8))
 (segment (start 117 62.5) (end 123.5 62.5) (width 0.5) (layer "B.Cu") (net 8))
 (segment (start 128 71.628) (end 131.826 71.628) (width 0.5) (layer "B.Cu") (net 8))
 (segment (start 127 66) (end 127 70.5) (width 0.5) (layer "B.Cu") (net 8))
 (segment (start 115.062 71.628) (end 115.062 65.786) (width 0.5) (layer "B.Cu") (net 8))
 (segment (start 139.192 73.426) (end 140.176 73.426) (width 0.5) (layer "B.Cu") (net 8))
 (segment (start 123.5 62.5) (end 127 66) (width 0.5) (layer "B.Cu") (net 8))
 (segment (start 140.256 78.994) (end 139.192 78.994) (width 0.5) (layer "B.Cu") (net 8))
 (segment (start 141 74.25) (end 141 78.25) (width 0.5) (layer "B.Cu") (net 8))
 (segment (start 140.176 73.426) (end 141 74.25) (width 0.5) (layer "B.Cu") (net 8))
 (segment (start 112.776 72.009) (end 114.681 72.009) (width 0.5) (layer "B.Cu") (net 8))
 (segment (start 122 90) (end 116.5 90) (width 0.5) (layer "B.Cu") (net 16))
 (segment (start 123 83) (end 123 89.40025) (width 0.5) (layer "B.Cu") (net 16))
 (segment (start 120.396 82.169) (end 122.169 82.169) (width 0.5) (layer "B.Cu") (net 16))
 (segment (start 122.169 82.169) (end 123 83) (width 0.5) (layer "B.Cu") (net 16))
 (segment (start 116.5 90) (end 114.42 92.58) (width 0.5) (layer "B.Cu") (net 16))
 (segment (start 123 89.40025) (end 122 90) (width 0.5) (layer "B.Cu") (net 16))
 (segment (start 114.42 92.58) (end 114.42 95.25) (width 0.5) (layer "B.Cu") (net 16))
 (segment (start 107.91 86.146) (end 109.347 84.709) (width 0.5) (layer "B.Cu") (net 2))
 (segment (start 109.347 84.709) (end 112.776 84.709) (width 0.5) (layer "B.Cu") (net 2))
 (segment (start 104.902 86.146) (end 107.91 86.146) (width 0.5) (layer "B.Cu") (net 2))
 (segment (start 112.776 79.629) (end 116.459 79.629) (width 0.5) (layer "B.Cu") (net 12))
 (segment (start 122.936 64.77) (end 124.206 66.04) (width 0.5) (layer "B.Cu") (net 12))
 (segment (start 118.872 64.77) (end 122.936 64.77) (width 0.5) (layer "B.Cu") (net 12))
 (segment (start 124.206 66.04) (end 124.206 71.628) (width 0.5) (layer "B.Cu") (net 12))
 (segment (start 117.856 78.232) (end 117.856 65.786) (width 0.5) (layer "B.Cu") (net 12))
 (segment (start 116.459 79.629) (end 117.856 78.232) (width 0.5) (layer "B.Cu") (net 12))
 (segment (start 117.856 65.786) (end 118.872 64.77) (width 0.5) (layer "B.Cu") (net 12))
 (segment (start 103.25 91.75) (end 102.616 91.186) (width 0.5) (layer "B.Cu") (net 3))
 (segment (start 115 89.5) (end 113.5 91.75) (width 0.5) (layer "B.Cu") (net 3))
 (segment (start 120.396 84.709) (end 116.205 84.709) (width 0.5) (layer "B.Cu") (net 3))
 (segment (start 103.298 83.646) (end 104.902 83.646) (width 0.5) (layer "B.Cu") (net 3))
 (segment (start 115.062 85.852) (end 115 89.5) (width 0.5) (layer "B.Cu") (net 3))
 (segment (start 116.205 84.709) (end 115.062 85.852) (width 0.5) (layer "B.Cu") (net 3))
 (segment (start 102.616 84.328) (end 103.298 83.646) (width 0.5) (layer "B.Cu") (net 3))
 (segment (start 102.616 91.186) (end 102.616 84.328) (width 0.5) (layer "B.Cu") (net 3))
 (segment (start 113.5 91.75) (end 103.25 91.75) (width 0.5) (layer "B.Cu") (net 3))
 (segment (start 121.629 79.629) (end 128 86) (width 0.5) (layer "B.Cu") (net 17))
 (segment (start 123 91.5) (end 118 91.5) (width 0.5) (layer "B.Cu") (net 17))
 (segment (start 118 91.5) (end 116.92 92.5) (width 0.5) (layer "B.Cu") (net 17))
 (segment (start 128 86) (end 128 90) (width 0.5) (layer "B.Cu") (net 17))
 (segment (start 120.396 79.629) (end 121.629 79.629) (width 0.5) (layer "B.Cu") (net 17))
 (segment (start 116.92 92.5) (end 116.92 95.25) (width 0.5) (layer "B.Cu") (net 17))
 (segment (start 126.5 91.5) (end 123 91.5) (width 0.5) (layer "B.Cu") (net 17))
 (segment (start 128 90) (end 126.5 91.5) (width 0.5) (layer "B.Cu") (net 17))
 (segment (start 139.192 85.344) (end 138.684 84.836) (width 0.5) (layer "B.Cu") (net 7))
 (segment (start 141.75 82.75) (end 142.5 82) (width 0.5) (layer "B.Cu") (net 7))
 (segment (start 132.8 86.8) (end 132.81 86.81) (width 0.5) (layer "B.Cu") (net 7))
 (segment (start 148.6 76.4) (end 144.304 76.418) (width 0.5) (layer "B.Cu") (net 7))
 (segment (start 148.6 82) (end 148.6 76.4) (width 0.5) (layer "B.Cu") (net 7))
 (segment (start 134.62 84.836) (end 132.8 86.4) (width 0.5) (layer "B.Cu") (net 7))
 (segment (start 132.81 86.81) (end 132.81 88.4174) (width 0.5) (layer "B.Cu") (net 7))
 (segment (start 138.684 84.836) (end 134.62 84.836) (width 0.5) (layer "B.Cu") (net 7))
 (segment (start 141.75 85.25) (end 141.75 82.75) (width 0.5) (layer "B.Cu") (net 7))
 (segment (start 142.5 82) (end 148.6 82) (width 0.5) (layer "B.Cu") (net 7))
 (segment (start 139.192 86.614) (end 139.192 85.344) (width 0.5) (layer "B.Cu") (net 7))
 (segment (start 140.386 86.614) (end 141.75 85.25) (width 0.5) (layer "B.Cu") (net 7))
 (segment (start 132.8 86.4) (end 132.8 86.8) (width 0.5) (layer "B.Cu") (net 7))
 (segment (start 139.192 86.614) (end 140.386 86.614) (width 0.5) (layer "B.Cu") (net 7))
 (segment (start 109.728 91.948) (end 110.998 93.218) (width 0.5) (layer "F.Cu") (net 11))
 (segment (start 111.633 74.549) (end 109.728 76.454) (width 0.5) (layer "F.Cu") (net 11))
 (segment (start 124.42 93.686) (end 124.42 95.25) (width 0.5) (layer "F.Cu") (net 11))
 (segment (start 123.952 93.218) (end 124.42 93.686) (width 0.5) (layer "F.Cu") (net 11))
 (segment (start 110.998 93.218) (end 123.952 93.218) (width 0.5) (layer "F.Cu") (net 11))
 (segment (start 112.776 74.549) (end 111.633 74.549) (width 0.5) (layer "F.Cu") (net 11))
 (segment (start 109.728 76.454) (end 109.728 91.948) (width 0.5) (layer "F.Cu") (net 11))
 (segment (start 124.42 95.25) (end 133.35 95.25) (width 0.5) (layer "B.Cu") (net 11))
 (segment (start 133.35 95.25) (end 135.625 92.975) (width 0.5) (layer "B.Cu") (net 11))
 (segment (start 135.625 92.975) (end 135.625 86.62) (width 0.5) (layer "B.Cu") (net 11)))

